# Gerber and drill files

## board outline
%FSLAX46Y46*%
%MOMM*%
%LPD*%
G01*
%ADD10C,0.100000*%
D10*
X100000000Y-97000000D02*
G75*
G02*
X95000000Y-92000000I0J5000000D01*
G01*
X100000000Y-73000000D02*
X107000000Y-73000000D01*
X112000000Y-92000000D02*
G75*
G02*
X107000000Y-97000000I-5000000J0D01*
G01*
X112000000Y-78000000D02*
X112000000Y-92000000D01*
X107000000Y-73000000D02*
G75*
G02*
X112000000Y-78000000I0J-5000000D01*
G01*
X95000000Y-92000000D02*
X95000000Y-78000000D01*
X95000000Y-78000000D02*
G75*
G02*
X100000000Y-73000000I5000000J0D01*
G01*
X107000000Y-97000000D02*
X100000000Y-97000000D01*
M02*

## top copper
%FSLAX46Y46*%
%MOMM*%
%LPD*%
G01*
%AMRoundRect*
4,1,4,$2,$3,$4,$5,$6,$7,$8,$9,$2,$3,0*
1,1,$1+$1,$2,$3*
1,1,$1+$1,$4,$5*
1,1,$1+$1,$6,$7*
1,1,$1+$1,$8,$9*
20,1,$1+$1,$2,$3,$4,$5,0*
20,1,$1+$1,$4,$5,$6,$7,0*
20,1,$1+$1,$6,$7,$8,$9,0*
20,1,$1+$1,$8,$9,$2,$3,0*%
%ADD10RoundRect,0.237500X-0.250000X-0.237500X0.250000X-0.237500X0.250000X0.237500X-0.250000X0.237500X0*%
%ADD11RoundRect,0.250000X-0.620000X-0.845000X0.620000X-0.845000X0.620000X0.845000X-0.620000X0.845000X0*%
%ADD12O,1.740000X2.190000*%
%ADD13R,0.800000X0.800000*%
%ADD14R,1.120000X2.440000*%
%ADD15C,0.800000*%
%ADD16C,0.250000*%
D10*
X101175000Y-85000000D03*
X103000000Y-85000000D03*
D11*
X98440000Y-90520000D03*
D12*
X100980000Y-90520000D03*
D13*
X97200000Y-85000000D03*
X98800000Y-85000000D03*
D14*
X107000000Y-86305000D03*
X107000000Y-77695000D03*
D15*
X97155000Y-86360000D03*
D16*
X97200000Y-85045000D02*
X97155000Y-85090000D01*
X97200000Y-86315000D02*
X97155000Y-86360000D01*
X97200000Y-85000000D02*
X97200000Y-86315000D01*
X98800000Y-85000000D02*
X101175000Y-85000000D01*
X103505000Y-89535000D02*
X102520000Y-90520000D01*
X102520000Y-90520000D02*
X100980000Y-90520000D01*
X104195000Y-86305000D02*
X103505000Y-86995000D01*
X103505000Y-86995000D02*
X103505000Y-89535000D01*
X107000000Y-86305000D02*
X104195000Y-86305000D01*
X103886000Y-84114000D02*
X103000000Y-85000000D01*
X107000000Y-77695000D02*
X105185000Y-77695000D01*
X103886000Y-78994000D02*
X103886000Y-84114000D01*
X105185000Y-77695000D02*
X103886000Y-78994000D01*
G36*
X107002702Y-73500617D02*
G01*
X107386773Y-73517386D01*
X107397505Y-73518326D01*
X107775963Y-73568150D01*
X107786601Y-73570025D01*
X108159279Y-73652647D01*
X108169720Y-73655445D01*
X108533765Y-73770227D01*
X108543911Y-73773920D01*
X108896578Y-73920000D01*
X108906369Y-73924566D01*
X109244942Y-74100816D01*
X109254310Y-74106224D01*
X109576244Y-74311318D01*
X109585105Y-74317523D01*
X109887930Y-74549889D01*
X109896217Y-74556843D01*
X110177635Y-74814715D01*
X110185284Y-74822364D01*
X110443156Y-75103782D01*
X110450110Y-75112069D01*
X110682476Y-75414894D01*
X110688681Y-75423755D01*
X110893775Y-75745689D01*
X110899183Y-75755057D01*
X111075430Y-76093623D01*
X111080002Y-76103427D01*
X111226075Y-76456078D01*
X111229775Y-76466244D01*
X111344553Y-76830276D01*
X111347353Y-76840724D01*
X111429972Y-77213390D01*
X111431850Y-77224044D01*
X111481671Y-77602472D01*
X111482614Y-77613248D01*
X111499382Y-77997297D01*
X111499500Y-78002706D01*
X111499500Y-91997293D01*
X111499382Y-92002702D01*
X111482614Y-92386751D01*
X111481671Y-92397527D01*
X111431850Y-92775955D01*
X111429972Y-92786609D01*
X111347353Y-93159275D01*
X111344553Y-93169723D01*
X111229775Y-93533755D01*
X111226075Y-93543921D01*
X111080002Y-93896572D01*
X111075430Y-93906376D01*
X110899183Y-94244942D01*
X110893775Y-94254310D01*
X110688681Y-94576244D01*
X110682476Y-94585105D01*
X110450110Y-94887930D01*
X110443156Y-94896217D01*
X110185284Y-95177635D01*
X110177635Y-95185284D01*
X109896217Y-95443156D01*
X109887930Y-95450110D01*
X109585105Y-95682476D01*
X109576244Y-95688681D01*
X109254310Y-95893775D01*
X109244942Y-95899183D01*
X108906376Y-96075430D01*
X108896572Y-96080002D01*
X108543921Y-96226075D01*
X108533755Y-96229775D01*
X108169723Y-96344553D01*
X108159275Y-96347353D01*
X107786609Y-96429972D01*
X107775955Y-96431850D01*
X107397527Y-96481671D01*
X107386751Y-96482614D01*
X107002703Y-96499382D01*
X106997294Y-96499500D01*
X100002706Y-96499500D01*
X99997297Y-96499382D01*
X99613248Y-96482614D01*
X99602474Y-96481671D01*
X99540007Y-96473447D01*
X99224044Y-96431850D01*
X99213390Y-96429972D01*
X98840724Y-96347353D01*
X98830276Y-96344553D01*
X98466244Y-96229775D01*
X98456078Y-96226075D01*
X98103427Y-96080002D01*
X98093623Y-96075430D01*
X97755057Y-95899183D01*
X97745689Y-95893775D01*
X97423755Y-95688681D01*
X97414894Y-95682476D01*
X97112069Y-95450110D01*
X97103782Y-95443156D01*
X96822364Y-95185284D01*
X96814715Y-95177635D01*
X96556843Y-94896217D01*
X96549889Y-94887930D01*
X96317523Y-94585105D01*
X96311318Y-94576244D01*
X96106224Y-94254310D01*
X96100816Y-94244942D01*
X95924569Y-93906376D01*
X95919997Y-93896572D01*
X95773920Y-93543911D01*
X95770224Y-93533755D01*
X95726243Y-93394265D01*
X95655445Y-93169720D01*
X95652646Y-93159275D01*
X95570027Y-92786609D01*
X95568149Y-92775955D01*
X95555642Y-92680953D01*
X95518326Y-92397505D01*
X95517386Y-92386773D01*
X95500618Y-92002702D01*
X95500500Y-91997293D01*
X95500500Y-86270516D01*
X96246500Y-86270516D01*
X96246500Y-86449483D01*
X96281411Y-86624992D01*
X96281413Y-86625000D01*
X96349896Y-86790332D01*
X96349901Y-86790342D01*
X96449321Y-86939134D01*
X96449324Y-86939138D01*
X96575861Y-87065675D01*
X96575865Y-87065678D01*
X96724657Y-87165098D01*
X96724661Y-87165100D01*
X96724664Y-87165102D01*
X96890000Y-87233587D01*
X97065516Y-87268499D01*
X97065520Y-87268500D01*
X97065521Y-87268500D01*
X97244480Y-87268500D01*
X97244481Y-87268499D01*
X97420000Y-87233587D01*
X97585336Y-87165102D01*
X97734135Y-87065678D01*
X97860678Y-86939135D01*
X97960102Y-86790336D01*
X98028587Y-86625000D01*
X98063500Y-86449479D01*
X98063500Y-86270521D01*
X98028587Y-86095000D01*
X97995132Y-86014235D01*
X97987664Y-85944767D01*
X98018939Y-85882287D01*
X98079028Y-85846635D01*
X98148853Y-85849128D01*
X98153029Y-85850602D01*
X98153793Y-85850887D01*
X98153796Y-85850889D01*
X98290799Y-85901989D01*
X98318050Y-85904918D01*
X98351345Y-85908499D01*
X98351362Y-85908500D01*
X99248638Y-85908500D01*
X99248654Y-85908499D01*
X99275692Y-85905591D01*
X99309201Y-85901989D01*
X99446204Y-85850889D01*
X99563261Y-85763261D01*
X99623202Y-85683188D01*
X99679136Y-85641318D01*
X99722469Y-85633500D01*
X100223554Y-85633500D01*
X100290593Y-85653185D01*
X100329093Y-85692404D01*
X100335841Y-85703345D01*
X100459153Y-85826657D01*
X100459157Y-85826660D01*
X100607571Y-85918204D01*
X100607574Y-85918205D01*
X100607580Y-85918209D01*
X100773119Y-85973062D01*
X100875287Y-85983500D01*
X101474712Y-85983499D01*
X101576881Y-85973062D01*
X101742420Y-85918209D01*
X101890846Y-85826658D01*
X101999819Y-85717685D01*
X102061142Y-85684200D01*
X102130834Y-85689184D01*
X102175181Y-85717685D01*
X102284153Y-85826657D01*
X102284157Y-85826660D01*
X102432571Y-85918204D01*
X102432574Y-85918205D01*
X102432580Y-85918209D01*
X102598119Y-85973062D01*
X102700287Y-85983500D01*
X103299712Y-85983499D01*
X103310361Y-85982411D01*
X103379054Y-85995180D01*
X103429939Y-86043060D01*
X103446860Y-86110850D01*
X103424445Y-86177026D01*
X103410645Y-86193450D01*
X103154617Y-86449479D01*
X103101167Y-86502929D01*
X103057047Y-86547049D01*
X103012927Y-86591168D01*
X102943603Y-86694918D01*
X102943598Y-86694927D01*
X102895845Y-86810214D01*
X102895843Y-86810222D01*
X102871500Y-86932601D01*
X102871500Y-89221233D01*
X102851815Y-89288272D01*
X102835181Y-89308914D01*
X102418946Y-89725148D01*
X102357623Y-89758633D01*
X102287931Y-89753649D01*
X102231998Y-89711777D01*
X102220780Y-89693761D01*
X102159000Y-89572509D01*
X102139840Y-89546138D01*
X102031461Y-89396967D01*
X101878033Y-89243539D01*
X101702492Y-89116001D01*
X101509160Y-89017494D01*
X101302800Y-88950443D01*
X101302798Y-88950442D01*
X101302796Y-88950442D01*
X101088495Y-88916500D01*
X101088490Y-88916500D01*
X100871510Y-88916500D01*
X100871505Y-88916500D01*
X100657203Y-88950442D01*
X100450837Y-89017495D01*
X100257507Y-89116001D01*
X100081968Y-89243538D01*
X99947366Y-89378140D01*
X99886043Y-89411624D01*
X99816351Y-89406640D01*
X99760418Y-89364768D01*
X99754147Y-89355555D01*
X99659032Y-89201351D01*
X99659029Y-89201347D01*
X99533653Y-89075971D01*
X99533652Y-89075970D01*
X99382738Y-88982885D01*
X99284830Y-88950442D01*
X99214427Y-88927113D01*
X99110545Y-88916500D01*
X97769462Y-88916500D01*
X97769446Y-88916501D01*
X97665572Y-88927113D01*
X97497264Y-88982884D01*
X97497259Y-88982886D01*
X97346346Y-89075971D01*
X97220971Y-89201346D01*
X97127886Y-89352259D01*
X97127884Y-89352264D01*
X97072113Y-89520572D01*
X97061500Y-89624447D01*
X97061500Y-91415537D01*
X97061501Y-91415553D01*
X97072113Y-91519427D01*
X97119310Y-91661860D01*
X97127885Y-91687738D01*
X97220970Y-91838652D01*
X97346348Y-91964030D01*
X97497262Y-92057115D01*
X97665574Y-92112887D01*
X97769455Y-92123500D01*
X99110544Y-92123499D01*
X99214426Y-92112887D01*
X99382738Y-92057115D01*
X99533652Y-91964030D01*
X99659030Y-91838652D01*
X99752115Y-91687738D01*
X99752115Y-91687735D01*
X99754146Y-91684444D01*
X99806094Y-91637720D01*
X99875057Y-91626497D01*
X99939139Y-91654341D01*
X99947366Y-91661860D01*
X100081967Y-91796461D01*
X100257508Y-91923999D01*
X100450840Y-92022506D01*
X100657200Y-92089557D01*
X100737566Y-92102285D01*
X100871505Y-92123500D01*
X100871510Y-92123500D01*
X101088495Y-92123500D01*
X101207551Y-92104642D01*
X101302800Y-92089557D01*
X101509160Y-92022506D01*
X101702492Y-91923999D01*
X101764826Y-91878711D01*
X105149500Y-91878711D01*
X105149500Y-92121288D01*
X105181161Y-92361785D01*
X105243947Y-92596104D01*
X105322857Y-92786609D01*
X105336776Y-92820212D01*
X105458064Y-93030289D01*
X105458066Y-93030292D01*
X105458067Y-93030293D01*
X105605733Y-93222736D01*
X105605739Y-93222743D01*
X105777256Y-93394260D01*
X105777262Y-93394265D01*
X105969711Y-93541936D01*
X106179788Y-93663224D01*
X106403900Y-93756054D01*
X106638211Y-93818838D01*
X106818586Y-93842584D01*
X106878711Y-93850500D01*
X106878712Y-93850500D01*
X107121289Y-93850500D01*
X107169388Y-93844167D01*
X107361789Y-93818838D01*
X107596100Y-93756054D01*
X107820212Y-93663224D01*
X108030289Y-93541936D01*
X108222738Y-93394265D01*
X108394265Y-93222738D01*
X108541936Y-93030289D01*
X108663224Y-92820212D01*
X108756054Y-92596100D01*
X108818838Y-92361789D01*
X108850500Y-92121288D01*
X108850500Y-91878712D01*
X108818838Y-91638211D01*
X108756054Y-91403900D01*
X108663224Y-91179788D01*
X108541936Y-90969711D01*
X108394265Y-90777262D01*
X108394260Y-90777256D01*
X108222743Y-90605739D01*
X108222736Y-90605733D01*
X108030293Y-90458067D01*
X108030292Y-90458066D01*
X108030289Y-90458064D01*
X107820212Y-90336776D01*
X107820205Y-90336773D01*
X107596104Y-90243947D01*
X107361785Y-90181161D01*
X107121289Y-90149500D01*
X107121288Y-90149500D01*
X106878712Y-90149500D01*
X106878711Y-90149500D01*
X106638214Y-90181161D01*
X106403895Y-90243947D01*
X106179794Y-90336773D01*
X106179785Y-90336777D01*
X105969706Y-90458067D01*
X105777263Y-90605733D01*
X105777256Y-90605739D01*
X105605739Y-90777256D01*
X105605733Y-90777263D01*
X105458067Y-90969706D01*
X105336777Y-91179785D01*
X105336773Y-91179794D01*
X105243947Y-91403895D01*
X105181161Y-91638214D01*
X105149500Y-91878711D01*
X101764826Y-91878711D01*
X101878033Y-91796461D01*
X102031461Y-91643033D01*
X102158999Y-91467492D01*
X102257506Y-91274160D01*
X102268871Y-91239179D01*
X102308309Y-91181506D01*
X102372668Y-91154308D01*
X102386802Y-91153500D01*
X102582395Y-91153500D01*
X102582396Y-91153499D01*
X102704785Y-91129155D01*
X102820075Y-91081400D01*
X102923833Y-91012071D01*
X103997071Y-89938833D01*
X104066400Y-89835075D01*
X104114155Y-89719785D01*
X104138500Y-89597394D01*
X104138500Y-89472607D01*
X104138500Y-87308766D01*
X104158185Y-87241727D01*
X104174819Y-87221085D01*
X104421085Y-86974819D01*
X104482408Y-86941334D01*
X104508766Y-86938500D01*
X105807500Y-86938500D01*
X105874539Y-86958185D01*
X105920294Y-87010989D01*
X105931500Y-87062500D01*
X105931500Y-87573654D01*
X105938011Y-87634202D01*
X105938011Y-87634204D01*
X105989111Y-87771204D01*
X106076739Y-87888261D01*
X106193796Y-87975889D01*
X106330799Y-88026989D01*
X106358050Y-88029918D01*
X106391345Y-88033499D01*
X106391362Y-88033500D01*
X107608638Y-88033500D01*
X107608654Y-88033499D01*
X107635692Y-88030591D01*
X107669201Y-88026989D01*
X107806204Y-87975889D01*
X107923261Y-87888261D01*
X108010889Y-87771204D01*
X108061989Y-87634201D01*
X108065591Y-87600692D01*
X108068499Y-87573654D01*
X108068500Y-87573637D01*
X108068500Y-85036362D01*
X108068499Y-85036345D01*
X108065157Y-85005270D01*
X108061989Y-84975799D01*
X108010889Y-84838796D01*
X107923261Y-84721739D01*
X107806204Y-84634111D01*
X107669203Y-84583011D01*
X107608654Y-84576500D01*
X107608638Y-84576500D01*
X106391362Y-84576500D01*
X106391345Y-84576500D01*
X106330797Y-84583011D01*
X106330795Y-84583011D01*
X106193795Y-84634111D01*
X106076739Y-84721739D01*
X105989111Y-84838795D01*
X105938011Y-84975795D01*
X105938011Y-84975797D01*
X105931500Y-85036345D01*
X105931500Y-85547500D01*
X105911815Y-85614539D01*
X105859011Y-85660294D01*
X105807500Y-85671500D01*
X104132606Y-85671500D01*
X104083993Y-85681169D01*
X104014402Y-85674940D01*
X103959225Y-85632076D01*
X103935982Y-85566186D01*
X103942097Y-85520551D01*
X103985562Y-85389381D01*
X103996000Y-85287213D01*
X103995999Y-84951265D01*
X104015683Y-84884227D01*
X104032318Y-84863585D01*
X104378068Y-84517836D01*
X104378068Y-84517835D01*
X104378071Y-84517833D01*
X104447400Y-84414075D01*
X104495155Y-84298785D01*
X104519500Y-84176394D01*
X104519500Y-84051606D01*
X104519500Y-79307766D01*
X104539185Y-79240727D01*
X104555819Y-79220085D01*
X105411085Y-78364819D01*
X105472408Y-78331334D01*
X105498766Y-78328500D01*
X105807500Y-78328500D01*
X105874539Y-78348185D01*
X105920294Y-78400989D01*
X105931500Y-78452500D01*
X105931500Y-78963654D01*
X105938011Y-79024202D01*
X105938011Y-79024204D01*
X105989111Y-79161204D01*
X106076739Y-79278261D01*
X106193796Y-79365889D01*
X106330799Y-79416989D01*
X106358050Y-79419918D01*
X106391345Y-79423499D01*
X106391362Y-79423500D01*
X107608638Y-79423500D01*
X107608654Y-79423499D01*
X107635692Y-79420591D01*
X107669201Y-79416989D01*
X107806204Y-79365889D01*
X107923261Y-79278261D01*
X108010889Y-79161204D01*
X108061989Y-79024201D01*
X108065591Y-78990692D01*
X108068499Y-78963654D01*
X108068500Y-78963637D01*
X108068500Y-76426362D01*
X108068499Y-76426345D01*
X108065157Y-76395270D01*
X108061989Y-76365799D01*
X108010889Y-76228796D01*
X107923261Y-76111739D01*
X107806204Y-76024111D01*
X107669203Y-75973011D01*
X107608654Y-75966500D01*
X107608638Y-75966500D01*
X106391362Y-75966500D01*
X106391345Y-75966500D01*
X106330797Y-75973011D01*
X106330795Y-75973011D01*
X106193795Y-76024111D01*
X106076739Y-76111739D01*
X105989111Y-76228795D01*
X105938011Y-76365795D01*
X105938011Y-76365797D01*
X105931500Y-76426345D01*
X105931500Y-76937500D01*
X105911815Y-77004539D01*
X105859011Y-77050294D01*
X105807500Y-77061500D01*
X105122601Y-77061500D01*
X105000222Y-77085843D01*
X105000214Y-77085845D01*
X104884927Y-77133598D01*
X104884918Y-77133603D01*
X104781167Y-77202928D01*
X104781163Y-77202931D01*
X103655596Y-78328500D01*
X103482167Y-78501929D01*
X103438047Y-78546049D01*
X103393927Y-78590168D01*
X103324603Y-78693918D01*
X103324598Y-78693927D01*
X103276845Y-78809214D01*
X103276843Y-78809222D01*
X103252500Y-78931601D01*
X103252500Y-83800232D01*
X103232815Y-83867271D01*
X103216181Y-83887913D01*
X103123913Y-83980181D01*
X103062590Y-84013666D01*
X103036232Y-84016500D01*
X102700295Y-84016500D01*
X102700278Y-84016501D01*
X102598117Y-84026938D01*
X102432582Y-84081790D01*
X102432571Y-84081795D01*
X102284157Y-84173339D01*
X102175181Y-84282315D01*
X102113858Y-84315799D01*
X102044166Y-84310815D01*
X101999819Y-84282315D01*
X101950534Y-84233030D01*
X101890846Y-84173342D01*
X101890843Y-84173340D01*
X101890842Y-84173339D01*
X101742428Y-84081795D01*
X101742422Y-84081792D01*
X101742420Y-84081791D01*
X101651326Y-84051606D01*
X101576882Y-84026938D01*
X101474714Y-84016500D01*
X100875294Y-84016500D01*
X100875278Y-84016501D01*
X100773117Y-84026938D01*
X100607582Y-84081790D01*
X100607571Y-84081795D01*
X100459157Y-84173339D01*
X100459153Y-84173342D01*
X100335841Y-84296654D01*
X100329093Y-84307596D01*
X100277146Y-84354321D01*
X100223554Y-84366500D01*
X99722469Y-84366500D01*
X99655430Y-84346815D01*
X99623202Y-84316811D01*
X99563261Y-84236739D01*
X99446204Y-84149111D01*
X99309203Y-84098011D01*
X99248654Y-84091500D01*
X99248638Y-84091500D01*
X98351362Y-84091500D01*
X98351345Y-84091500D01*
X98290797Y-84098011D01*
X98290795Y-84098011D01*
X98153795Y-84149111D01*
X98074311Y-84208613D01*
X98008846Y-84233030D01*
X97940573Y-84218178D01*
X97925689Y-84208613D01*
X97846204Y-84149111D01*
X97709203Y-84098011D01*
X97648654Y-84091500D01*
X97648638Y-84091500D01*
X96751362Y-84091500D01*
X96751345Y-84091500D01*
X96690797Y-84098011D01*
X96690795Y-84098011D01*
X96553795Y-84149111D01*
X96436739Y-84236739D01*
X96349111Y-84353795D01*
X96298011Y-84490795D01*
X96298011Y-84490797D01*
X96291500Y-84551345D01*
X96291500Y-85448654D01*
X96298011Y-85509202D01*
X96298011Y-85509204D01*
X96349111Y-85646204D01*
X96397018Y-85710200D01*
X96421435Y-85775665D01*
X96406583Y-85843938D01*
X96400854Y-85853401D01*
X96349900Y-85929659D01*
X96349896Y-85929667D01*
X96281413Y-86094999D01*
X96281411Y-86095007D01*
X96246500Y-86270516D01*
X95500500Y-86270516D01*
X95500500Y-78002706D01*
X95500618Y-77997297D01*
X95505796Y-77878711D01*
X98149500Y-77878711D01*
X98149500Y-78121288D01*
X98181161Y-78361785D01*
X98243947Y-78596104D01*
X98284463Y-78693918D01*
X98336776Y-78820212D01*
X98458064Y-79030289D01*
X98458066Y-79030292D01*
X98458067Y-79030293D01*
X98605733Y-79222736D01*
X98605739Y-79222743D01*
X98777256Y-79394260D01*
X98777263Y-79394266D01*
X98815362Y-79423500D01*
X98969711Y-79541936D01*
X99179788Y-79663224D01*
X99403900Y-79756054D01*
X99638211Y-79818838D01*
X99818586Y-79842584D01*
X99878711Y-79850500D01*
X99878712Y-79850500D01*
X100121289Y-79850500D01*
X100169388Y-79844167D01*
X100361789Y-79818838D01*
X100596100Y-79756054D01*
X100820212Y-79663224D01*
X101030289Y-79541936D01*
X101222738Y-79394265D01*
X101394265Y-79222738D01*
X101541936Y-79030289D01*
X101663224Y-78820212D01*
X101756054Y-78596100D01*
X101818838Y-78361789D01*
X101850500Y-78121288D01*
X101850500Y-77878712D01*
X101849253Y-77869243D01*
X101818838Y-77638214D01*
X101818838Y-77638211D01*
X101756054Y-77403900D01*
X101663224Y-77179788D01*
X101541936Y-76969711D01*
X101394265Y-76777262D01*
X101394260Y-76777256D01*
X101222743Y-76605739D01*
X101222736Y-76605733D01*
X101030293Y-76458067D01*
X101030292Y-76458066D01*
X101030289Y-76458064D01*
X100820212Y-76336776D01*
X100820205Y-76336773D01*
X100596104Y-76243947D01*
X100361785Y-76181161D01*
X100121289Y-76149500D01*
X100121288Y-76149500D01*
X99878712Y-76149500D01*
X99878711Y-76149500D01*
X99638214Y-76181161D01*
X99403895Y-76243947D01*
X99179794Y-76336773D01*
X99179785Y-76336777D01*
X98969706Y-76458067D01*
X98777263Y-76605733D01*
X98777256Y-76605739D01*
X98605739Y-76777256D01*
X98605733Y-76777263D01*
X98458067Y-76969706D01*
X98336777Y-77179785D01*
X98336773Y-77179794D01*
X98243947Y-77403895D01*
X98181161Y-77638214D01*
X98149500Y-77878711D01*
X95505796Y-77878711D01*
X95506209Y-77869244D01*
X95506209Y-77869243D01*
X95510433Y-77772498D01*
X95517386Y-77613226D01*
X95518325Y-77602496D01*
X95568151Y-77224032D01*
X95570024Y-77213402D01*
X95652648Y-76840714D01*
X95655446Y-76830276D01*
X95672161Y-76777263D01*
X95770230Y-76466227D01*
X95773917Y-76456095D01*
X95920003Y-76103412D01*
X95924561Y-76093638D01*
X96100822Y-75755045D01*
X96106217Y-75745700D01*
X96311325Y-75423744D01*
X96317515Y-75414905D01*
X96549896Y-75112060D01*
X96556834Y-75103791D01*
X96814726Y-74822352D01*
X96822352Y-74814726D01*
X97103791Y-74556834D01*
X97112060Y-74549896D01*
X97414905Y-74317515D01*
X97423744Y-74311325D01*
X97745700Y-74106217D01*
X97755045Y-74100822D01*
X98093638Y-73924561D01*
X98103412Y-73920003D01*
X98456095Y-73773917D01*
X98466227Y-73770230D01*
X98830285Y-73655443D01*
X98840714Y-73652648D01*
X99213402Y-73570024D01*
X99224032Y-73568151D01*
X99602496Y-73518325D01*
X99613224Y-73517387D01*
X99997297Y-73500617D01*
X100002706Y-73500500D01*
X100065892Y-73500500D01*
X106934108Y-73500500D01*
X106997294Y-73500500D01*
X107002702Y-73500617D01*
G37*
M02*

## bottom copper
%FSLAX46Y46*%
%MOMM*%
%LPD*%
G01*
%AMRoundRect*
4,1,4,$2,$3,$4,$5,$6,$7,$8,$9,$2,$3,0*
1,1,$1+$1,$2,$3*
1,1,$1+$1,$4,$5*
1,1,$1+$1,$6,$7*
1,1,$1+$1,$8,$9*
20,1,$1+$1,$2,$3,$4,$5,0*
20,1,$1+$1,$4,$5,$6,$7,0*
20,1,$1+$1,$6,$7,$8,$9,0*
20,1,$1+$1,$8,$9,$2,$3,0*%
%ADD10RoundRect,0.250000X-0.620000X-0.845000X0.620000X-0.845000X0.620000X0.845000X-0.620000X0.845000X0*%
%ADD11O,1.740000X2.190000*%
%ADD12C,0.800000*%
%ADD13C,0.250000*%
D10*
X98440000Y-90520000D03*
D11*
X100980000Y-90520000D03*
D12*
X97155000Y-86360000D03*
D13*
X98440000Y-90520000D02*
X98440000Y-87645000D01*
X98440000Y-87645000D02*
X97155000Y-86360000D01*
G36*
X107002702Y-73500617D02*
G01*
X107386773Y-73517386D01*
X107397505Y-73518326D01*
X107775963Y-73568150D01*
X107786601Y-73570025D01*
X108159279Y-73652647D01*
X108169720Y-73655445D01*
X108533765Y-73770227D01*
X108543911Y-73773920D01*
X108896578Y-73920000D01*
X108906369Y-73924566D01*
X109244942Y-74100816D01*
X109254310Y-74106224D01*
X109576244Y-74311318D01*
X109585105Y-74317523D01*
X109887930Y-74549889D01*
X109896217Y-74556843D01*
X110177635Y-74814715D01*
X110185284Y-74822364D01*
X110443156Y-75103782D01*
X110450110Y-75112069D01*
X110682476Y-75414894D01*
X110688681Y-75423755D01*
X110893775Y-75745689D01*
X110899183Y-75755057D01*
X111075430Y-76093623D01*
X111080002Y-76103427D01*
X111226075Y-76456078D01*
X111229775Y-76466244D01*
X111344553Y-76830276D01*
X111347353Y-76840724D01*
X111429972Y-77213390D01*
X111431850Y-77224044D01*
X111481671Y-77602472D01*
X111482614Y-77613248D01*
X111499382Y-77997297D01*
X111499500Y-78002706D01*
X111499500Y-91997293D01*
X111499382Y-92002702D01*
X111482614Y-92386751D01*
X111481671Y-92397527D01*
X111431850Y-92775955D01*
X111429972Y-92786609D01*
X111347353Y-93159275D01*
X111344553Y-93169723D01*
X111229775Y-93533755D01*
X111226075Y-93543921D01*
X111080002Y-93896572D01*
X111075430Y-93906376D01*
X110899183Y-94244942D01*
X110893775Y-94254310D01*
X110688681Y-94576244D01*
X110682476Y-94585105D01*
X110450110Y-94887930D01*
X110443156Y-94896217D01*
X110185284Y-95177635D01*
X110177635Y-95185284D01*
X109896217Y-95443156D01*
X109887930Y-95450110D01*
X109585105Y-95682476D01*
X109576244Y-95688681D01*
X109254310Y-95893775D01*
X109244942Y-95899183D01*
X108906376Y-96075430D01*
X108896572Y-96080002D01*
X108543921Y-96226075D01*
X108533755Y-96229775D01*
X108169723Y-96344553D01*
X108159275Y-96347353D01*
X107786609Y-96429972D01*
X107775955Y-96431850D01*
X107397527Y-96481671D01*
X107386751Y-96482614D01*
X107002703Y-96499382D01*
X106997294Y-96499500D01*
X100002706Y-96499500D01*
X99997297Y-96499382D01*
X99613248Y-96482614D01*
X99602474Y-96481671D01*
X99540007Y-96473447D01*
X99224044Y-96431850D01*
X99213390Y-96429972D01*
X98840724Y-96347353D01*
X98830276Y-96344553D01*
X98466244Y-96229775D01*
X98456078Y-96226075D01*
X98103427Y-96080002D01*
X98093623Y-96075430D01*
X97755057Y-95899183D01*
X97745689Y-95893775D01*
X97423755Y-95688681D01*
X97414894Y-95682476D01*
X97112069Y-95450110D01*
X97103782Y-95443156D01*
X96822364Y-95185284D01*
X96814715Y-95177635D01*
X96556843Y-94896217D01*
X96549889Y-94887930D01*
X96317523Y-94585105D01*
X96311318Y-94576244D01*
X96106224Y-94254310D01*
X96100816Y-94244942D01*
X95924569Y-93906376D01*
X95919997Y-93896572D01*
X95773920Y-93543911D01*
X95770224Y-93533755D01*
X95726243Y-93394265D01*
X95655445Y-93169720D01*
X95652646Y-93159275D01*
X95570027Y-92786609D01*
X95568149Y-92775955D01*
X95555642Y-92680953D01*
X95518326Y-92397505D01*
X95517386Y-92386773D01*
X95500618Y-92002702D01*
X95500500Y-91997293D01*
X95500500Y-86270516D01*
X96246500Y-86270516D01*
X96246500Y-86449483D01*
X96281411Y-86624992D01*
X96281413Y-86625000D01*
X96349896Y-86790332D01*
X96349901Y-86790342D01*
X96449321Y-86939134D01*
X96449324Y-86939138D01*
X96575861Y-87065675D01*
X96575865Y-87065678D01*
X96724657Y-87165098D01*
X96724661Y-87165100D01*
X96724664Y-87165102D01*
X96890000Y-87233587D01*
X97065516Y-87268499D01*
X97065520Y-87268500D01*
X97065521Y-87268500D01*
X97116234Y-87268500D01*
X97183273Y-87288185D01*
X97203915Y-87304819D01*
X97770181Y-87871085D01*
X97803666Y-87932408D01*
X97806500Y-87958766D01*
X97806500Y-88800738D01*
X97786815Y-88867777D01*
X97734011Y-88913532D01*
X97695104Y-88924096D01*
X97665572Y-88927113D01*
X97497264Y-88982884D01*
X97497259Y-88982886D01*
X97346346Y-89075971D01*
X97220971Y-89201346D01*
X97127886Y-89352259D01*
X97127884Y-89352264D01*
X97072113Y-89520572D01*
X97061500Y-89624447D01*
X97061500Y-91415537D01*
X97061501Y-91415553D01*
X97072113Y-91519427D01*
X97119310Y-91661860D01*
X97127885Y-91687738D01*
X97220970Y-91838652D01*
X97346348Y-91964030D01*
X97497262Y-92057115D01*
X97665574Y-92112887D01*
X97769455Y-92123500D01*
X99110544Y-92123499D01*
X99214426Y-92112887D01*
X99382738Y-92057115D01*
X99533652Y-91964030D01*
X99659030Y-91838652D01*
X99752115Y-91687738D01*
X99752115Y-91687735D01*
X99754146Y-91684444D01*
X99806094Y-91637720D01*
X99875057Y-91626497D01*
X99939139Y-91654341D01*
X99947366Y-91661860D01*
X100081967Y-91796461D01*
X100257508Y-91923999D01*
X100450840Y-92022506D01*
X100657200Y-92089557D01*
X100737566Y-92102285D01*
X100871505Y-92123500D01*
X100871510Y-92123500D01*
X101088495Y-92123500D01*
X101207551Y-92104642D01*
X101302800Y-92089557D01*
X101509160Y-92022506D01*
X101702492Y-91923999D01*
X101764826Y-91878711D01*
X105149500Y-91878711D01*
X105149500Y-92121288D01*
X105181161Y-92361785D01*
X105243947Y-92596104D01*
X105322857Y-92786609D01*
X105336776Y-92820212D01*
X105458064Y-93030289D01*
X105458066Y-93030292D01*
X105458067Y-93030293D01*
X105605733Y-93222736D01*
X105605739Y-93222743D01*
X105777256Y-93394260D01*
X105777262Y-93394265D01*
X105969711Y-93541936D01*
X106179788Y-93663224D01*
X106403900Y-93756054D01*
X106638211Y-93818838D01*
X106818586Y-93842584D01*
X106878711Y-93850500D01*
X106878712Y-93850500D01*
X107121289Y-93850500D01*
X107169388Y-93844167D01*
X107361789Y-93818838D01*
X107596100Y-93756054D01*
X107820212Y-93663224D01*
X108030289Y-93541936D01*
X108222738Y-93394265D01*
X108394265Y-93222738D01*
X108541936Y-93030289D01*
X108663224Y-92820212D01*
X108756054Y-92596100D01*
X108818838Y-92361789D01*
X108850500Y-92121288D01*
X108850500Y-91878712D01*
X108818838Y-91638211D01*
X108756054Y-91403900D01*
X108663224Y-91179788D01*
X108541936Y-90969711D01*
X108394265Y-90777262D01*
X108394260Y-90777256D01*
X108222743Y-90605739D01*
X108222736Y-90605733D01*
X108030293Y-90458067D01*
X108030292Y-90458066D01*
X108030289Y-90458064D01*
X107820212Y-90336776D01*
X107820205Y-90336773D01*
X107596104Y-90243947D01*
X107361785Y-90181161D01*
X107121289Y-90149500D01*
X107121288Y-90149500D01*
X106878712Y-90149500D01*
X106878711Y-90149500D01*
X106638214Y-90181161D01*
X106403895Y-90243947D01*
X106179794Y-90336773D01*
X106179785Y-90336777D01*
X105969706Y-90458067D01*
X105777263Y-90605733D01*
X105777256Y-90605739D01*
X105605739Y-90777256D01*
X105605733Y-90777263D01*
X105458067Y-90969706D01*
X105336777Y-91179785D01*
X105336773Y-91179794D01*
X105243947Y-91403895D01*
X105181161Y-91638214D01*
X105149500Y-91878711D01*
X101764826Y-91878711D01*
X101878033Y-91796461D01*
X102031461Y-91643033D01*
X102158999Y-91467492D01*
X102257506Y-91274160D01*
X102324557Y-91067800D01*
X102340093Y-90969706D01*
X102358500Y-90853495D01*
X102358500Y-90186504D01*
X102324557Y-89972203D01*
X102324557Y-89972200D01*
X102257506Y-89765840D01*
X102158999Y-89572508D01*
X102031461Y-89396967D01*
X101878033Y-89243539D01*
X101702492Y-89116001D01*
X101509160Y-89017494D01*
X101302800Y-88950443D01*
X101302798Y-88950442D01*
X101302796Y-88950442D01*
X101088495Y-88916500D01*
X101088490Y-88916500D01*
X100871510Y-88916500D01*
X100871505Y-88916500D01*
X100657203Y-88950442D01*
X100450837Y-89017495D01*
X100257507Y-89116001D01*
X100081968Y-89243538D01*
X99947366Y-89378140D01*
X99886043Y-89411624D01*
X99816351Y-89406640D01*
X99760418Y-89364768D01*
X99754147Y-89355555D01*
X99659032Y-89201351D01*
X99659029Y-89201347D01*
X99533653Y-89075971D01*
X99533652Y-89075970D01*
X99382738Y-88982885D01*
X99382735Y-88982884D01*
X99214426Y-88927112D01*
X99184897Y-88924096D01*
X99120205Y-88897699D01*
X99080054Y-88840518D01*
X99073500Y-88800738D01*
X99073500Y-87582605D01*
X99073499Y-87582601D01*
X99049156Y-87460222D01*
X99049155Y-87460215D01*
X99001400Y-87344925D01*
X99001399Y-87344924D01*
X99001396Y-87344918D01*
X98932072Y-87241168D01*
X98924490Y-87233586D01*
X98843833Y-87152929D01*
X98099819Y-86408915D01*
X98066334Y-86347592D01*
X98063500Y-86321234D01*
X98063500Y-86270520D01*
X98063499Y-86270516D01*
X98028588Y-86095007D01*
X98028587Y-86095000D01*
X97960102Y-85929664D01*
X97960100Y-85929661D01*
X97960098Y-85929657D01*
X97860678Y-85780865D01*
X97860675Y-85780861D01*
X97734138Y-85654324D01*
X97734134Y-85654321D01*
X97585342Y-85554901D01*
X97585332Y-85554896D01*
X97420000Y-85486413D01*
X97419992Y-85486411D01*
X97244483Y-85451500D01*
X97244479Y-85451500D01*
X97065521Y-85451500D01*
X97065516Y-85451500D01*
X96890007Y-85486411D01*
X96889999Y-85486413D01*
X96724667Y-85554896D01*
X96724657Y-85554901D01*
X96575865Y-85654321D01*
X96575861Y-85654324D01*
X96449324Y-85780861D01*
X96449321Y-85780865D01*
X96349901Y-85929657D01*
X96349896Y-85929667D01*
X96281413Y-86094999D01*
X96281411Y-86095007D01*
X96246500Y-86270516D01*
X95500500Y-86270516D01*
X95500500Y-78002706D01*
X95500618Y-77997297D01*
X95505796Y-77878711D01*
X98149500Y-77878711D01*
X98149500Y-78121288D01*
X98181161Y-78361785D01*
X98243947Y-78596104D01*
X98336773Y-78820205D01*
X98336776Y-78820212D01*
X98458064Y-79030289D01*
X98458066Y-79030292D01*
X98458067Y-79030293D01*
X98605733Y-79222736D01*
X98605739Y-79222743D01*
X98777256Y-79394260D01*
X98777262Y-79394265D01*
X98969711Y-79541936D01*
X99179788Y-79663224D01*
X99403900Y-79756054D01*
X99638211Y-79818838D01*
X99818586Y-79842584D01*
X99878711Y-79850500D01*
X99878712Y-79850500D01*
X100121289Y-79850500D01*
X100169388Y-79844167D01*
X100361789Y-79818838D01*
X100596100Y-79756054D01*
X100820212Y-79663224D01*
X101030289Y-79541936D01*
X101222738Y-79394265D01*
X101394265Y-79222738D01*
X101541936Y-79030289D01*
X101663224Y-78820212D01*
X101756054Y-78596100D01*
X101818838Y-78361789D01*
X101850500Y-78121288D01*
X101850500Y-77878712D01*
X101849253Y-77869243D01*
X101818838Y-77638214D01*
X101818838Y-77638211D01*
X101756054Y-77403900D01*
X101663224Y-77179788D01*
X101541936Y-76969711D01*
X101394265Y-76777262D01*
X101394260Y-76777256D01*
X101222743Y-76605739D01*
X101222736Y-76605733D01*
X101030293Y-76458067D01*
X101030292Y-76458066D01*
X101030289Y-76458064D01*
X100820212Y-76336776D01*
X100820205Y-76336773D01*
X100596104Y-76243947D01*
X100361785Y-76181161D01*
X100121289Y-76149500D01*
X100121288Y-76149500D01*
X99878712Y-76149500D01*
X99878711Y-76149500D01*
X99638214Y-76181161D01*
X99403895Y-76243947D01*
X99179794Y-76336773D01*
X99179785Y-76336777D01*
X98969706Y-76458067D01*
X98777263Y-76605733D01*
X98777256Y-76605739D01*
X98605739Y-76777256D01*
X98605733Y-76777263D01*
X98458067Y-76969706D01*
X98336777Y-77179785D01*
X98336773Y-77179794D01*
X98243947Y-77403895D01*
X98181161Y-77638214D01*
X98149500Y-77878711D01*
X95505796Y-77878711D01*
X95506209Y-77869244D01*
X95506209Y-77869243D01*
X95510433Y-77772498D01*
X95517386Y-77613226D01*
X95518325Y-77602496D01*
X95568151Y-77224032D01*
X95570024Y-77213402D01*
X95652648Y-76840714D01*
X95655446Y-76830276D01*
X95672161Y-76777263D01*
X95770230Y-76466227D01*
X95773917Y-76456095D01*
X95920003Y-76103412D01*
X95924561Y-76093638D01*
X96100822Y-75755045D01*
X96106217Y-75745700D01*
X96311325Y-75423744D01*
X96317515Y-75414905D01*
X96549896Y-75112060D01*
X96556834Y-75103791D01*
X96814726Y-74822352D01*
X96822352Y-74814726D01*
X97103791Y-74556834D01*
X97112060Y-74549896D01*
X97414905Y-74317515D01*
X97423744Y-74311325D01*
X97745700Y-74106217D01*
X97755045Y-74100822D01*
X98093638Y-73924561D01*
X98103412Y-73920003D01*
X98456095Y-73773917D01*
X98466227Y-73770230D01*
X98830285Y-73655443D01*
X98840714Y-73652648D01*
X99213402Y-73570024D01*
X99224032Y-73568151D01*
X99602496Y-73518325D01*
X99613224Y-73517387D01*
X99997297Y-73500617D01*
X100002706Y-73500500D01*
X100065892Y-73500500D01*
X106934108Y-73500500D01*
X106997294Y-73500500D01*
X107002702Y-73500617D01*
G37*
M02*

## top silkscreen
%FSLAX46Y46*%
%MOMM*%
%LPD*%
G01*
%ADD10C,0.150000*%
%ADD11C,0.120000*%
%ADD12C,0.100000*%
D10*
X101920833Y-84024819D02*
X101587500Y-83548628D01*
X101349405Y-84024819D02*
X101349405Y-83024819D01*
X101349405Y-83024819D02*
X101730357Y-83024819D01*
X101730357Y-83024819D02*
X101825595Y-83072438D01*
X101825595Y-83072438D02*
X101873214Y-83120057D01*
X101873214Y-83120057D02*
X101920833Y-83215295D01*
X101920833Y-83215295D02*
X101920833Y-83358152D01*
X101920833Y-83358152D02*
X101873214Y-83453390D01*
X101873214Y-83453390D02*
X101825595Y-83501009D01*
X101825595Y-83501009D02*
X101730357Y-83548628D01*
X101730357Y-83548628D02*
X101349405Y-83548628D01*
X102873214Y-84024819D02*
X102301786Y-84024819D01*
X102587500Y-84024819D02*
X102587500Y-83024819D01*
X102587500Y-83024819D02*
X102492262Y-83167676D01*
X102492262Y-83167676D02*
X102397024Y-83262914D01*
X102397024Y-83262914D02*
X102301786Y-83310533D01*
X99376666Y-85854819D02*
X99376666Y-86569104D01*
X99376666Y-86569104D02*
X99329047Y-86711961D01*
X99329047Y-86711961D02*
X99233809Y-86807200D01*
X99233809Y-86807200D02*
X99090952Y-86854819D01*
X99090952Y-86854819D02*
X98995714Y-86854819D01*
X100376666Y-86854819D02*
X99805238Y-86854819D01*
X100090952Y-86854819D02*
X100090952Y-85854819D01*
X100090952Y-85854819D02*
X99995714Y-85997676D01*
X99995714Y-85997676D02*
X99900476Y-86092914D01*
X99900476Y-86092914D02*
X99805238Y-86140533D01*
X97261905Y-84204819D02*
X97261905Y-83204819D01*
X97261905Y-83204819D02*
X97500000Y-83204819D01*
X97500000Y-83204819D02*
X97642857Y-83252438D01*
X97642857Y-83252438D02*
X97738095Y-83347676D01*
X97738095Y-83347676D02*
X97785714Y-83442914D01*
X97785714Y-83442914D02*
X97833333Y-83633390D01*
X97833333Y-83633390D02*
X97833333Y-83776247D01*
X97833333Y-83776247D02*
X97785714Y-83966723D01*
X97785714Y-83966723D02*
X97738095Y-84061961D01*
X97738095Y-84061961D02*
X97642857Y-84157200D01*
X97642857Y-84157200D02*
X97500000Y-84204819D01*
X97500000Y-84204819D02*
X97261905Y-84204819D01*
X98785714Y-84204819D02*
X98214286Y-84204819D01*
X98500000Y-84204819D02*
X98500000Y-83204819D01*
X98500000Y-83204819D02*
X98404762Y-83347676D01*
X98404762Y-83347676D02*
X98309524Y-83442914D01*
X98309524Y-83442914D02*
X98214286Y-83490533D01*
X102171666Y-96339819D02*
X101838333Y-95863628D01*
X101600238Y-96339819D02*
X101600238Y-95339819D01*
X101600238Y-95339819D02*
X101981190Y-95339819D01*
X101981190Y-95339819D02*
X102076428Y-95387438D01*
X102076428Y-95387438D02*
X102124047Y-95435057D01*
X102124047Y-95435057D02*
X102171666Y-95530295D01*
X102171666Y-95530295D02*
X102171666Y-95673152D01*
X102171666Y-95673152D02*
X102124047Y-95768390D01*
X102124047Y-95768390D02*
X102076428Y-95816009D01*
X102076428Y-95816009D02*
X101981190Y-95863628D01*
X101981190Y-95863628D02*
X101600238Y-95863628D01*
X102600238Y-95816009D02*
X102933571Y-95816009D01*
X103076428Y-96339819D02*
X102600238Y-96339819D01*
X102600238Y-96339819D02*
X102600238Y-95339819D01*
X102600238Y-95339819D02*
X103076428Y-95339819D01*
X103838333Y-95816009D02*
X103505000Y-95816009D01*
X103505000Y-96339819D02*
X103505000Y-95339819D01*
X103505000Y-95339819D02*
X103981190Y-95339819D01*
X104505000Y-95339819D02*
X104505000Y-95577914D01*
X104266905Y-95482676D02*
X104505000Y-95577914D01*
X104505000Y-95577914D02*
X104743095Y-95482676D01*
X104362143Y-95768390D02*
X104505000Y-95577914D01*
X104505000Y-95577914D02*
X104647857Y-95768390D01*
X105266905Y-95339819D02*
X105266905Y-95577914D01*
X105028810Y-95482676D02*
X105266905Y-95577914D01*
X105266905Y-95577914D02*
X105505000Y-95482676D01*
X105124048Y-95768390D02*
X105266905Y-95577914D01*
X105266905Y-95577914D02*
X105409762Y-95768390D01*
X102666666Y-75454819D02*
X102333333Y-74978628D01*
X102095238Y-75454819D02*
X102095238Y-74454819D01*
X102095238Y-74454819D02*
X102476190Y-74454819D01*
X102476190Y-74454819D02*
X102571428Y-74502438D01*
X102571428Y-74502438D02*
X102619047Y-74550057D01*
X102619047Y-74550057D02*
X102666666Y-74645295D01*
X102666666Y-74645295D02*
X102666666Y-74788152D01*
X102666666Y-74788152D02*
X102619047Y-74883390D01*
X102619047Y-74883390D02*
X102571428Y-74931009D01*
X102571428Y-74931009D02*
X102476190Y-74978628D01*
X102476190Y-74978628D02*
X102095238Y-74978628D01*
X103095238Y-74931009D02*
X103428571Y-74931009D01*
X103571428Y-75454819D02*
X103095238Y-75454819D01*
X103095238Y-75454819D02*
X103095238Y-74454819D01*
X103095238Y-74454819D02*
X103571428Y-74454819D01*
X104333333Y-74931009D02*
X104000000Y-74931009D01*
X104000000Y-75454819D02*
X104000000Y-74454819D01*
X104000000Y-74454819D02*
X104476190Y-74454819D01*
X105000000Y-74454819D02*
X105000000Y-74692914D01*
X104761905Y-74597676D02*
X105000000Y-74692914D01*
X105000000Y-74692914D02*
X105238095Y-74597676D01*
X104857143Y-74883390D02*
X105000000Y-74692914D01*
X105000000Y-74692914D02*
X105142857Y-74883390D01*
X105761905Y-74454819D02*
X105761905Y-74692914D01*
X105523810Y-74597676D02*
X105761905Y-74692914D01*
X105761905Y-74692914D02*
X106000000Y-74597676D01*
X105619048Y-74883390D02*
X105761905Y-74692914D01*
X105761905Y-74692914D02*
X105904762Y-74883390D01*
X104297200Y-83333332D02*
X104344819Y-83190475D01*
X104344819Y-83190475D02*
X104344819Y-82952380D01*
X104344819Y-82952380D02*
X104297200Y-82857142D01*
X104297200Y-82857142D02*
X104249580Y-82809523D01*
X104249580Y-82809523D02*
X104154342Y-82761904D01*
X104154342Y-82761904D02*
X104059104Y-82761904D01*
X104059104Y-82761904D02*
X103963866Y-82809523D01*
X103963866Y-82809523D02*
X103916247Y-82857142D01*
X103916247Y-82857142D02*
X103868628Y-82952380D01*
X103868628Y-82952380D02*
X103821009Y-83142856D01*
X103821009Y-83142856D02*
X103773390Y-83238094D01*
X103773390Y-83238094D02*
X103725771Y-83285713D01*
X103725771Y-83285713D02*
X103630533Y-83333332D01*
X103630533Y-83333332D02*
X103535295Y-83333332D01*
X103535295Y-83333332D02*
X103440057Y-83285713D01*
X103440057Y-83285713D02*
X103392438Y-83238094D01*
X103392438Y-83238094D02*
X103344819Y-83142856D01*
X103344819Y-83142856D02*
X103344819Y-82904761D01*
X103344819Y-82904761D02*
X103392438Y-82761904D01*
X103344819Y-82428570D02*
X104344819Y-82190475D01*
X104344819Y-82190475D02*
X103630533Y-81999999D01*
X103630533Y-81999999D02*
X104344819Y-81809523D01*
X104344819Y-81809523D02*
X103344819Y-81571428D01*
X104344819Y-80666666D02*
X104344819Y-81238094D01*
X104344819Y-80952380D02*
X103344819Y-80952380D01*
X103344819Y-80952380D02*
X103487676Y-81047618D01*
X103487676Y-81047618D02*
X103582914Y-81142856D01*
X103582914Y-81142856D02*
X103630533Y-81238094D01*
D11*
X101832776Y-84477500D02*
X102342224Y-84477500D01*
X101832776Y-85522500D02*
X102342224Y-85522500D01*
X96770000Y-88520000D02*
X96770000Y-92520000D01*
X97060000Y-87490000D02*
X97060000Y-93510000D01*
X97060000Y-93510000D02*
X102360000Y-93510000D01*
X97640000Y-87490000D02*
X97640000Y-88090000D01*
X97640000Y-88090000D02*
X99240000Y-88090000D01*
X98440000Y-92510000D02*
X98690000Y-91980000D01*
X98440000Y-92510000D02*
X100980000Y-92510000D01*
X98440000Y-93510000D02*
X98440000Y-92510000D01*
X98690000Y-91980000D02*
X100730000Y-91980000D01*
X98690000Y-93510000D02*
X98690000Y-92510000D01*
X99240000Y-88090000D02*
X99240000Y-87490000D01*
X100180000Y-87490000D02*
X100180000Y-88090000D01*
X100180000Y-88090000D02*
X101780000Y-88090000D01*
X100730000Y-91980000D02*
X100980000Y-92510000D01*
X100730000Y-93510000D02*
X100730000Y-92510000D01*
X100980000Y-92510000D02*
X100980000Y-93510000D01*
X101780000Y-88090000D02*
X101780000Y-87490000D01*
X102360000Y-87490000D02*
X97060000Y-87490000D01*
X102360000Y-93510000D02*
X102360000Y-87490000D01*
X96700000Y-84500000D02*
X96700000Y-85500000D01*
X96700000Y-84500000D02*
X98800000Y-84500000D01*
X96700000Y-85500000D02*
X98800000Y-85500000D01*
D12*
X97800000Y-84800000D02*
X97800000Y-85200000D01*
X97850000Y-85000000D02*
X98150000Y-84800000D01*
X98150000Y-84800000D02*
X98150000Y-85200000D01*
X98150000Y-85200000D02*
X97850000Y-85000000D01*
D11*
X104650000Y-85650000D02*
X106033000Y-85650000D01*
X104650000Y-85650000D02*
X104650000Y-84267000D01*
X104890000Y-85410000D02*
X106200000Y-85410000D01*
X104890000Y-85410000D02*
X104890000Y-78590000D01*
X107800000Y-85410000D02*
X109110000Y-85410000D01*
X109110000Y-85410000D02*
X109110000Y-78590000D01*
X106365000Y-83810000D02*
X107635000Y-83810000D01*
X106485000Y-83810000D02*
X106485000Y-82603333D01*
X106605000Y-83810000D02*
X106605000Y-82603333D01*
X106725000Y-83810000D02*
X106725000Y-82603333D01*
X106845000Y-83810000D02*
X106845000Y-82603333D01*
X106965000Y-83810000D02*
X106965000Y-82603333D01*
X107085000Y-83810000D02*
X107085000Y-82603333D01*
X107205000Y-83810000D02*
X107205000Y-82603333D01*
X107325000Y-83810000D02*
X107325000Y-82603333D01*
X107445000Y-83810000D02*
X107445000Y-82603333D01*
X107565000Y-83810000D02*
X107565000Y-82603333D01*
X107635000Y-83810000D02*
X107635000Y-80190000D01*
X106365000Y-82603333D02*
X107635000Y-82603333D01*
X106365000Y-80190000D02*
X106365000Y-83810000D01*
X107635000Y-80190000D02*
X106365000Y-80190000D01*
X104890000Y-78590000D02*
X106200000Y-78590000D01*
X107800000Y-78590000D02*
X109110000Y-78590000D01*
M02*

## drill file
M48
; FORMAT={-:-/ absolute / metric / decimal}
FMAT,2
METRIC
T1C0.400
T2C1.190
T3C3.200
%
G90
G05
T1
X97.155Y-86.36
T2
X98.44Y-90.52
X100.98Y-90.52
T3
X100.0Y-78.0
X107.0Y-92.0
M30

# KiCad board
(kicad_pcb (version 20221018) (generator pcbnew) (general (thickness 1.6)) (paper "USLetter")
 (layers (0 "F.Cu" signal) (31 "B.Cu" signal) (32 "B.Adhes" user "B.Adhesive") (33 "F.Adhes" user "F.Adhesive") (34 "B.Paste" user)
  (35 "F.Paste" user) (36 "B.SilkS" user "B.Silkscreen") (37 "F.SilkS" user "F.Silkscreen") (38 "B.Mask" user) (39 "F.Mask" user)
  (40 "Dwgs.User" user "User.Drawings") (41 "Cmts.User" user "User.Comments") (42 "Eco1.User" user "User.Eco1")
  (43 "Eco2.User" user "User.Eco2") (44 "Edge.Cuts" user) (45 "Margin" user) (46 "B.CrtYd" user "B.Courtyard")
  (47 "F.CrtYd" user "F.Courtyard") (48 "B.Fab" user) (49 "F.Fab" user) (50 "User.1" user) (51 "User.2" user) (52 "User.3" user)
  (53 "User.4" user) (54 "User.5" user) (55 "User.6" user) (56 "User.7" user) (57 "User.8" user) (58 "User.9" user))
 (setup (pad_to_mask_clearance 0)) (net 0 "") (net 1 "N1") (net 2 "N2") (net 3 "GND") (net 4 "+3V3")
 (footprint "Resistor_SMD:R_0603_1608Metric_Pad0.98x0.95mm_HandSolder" (layer "F.Cu") (at 102.0875 85)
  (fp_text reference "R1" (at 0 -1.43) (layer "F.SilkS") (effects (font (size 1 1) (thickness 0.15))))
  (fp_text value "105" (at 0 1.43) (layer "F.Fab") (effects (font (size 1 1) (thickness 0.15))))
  (fp_line (start -0.254724 -0.5225) (end 0.254724 -0.5225) (stroke (width 0.12) (type solid)) (layer "F.SilkS"))
  (fp_line (start -0.254724 0.5225) (end 0.254724 0.5225) (stroke (width 0.12) (type solid)) (layer "F.SilkS"))
  (pad "1" smd roundrect (at -0.9125 0) (size 0.975 0.95) (layers "F.Cu" "F.Paste" "F.Mask") (roundrect_rratio 0.25) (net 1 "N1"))
  (pad "2" smd roundrect (at 0.9125 0) (size 0.975 0.95) (layers "F.Cu" "F.Paste" "F.Mask") (roundrect_rratio 0.25) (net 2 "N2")))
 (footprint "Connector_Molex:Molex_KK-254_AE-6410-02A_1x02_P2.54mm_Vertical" (layer "F.Cu") (at 98.44 90.52)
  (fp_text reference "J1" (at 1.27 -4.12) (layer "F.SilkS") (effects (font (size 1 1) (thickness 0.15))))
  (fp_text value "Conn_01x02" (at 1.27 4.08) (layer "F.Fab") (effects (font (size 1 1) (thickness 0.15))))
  (fp_line (start -1.67 -2) (end -1.67 2) (stroke (width 0.12) (type solid)) (layer "F.SilkS"))
  (fp_line (start -1.38 -3.03) (end -1.38 2.99) (stroke (width 0.12) (type solid)) (layer "F.SilkS"))
  (fp_line (start -1.38 2.99) (end 3.92 2.99) (stroke (width 0.12) (type solid)) (layer "F.SilkS"))
  (fp_line (start -0.8 -3.03) (end -0.8 -2.43) (stroke (width 0.12) (type solid)) (layer "F.SilkS"))
  (fp_line (start -0.8 -2.43) (end 0.8 -2.43) (stroke (width 0.12) (type solid)) (layer "F.SilkS"))
  (fp_line (start 0 1.99) (end 0.25 1.46) (stroke (width 0.12) (type solid)) (layer "F.SilkS"))
  (fp_line (start 0 1.99) (end 2.54 1.99) (stroke (width 0.12) (type solid)) (layer "F.SilkS"))
  (fp_line (start 0 2.99) (end 0 1.99) (stroke (width 0.12) (type solid)) (layer "F.SilkS"))
  (fp_line (start 0.25 1.46) (end 2.29 1.46) (stroke (width 0.12) (type solid)) (layer "F.SilkS"))
  (fp_line (start 0.25 2.99) (end 0.25 1.99) (stroke (width 0.12) (type solid)) (layer "F.SilkS"))
  (fp_line (start 0.8 -2.43) (end 0.8 -3.03) (stroke (width 0.12) (type solid)) (layer "F.SilkS"))
  (fp_line (start 1.74 -3.03) (end 1.74 -2.43) (stroke (width 0.12) (type solid)) (layer "F.SilkS"))
  (fp_line (start 1.74 -2.43) (end 3.34 -2.43) (stroke (width 0.12) (type solid)) (layer "F.SilkS"))
  (fp_line (start 2.29 1.46) (end 2.54 1.99) (stroke (width 0.12) (type solid)) (layer "F.SilkS"))
  (fp_line (start 2.29 2.99) (end 2.29 1.99) (stroke (width 0.12) (type solid)) (layer "F.SilkS"))
  (fp_line (start 2.54 1.99) (end 2.54 2.99) (stroke (width 0.12) (type solid)) (layer "F.SilkS"))
  (fp_line (start 3.34 -2.43) (end 3.34 -3.03) (stroke (width 0.12) (type solid)) (layer "F.SilkS"))
  (fp_line (start 3.92 -3.03) (end -1.38 -3.03) (stroke (width 0.12) (type solid)) (layer "F.SilkS"))
  (fp_line (start 3.92 2.99) (end 3.92 -3.03) (stroke (width 0.12) (type solid)) (layer "F.SilkS"))
  (pad "1" thru_hole roundrect (at 0 0) (size 1.74 2.19) (drill 1.19) (layers "*.Cu" "*.Mask") (roundrect_rratio 0.143678) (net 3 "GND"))
  (pad "2" thru_hole oval (at 2.54 0) (size 1.74 2.19) (drill 1.19) (layers "*.Cu" "*.Mask") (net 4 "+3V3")))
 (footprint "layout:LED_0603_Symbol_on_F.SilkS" (layer "F.Cu") (at 98 85)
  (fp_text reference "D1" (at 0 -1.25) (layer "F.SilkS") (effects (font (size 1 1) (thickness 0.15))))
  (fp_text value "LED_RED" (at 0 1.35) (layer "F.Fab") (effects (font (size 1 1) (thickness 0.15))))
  (fp_line (start -1.3 -0.5) (end -1.3 0.5) (stroke (width 0.12) (type solid)) (layer "F.SilkS"))
  (fp_line (start -1.3 -0.5) (end 0.8 -0.5) (stroke (width 0.12) (type solid)) (layer "F.SilkS"))
  (fp_line (start -1.3 0.5) (end 0.8 0.5) (stroke (width 0.12) (type solid)) (layer "F.SilkS"))
  (fp_line (start -0.2 -0.2) (end -0.2 0.2) (stroke (width 0.1) (type solid)) (layer "F.SilkS"))
  (fp_line (start -0.15 0) (end 0.15 -0.2) (stroke (width 0.1) (type solid)) (layer "F.SilkS"))
  (fp_line (start 0.15 -0.2) (end 0.15 0.2) (stroke (width 0.1) (type solid)) (layer "F.SilkS"))
  (fp_line (start 0.15 0.2) (end -0.15 0) (stroke (width 0.1) (type solid)) (layer "F.SilkS"))
  (pad "1" smd rect (at -0.8 0 180) (size 0.8 0.8) (layers "F.Cu" "F.Paste" "F.Mask") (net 3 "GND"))
  (pad "2" smd rect (at 0.8 0 180) (size 0.8 0.8) (layers "F.Cu" "F.Paste" "F.Mask") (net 1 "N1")))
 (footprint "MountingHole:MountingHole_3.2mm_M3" (layer "F.Cu") (at 107 92)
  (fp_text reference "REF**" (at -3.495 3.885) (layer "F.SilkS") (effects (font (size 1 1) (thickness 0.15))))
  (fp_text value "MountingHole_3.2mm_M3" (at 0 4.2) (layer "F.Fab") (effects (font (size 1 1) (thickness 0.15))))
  (pad "" np_thru_hole circle (at 0 0) (size 3.2 3.2) (drill 3.2) (layers "F&B.Cu" "*.Mask")))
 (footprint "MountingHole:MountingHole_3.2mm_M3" (layer "F.Cu") (at 100 78)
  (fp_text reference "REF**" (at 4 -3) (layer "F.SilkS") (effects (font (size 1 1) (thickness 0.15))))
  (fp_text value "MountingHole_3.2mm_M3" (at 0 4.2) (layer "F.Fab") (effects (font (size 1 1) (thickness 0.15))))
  (pad "" np_thru_hole circle (at 0 0) (size 3.2 3.2) (drill 3.2) (layers "*.Cu" "*.Mask")))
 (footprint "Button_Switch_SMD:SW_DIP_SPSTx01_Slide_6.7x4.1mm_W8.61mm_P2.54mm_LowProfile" (layer "F.Cu") (at 107 82 90)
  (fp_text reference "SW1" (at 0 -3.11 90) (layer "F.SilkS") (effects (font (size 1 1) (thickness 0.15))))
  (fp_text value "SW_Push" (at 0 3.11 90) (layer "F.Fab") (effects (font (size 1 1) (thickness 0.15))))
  (fp_line (start -3.65 -2.35) (end -3.65 -0.967) (stroke (width 0.12) (type solid)) (layer "F.SilkS"))
  (fp_line (start -3.65 -2.35) (end -2.267 -2.35) (stroke (width 0.12) (type solid)) (layer "F.SilkS"))
  (fp_line (start -3.41 -2.11) (end -3.41 -0.8) (stroke (width 0.12) (type solid)) (layer "F.SilkS"))
  (fp_line (start -3.41 -2.11) (end 3.41 -2.11) (stroke (width 0.12) (type solid)) (layer "F.SilkS"))
  (fp_line (start -3.41 0.8) (end -3.41 2.11) (stroke (width 0.12) (type solid)) (layer "F.SilkS"))
  (fp_line (start -3.41 2.11) (end 3.41 2.11) (stroke (width 0.12) (type solid)) (layer "F.SilkS"))
  (fp_line (start -1.81 -0.635) (end -1.81 0.635) (stroke (width 0.12) (type solid)) (layer "F.SilkS"))
  (fp_line (start -1.81 -0.515) (end -0.603333 -0.515) (stroke (width 0.12) (type solid)) (layer "F.SilkS"))
  (fp_line (start -1.81 -0.395) (end -0.603333 -0.395) (stroke (width 0.12) (type solid)) (layer "F.SilkS"))
  (fp_line (start -1.81 -0.275) (end -0.603333 -0.275) (stroke (width 0.12) (type solid)) (layer "F.SilkS"))
  (fp_line (start -1.81 -0.155) (end -0.603333 -0.155) (stroke (width 0.12) (type solid)) (layer "F.SilkS"))
  (fp_line (start -1.81 -0.035) (end -0.603333 -0.035) (stroke (width 0.12) (type solid)) (layer "F.SilkS"))
  (fp_line (start -1.81 0.085) (end -0.603333 0.085) (stroke (width 0.12) (type solid)) (layer "F.SilkS"))
  (fp_line (start -1.81 0.205) (end -0.603333 0.205) (stroke (width 0.12) (type solid)) (layer "F.SilkS"))
  (fp_line (start -1.81 0.325) (end -0.603333 0.325) (stroke (width 0.12) (type solid)) (layer "F.SilkS"))
  (fp_line (start -1.81 0.445) (end -0.603333 0.445) (stroke (width 0.12) (type solid)) (layer "F.SilkS"))
  (fp_line (start -1.81 0.565) (end -0.603333 0.565) (stroke (width 0.12) (type solid)) (layer "F.SilkS"))
  (fp_line (start -1.81 0.635) (end 1.81 0.635) (stroke (width 0.12) (type solid)) (layer "F.SilkS"))
  (fp_line (start -0.603333 -0.635) (end -0.603333 0.635) (stroke (width 0.12) (type solid)) (layer "F.SilkS"))
  (fp_line (start 1.81 -0.635) (end -1.81 -0.635) (stroke (width 0.12) (type solid)) (layer "F.SilkS"))
  (fp_line (start 1.81 0.635) (end 1.81 -0.635) (stroke (width 0.12) (type solid)) (layer "F.SilkS"))
  (fp_line (start 3.41 -2.11) (end 3.41 -0.8) (stroke (width 0.12) (type solid)) (layer "F.SilkS"))
  (fp_line (start 3.41 0.8) (end 3.41 2.11) (stroke (width 0.12) (type solid)) (layer "F.SilkS"))
  (pad "1" smd rect (at -4.305 0 90) (size 2.44 1.12) (layers "F.Cu" "F.Paste" "F.Mask") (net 4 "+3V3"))
  (pad "2" smd rect (at 4.305 0 90) (size 2.44 1.12) (layers "F.Cu" "F.Paste" "F.Mask") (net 2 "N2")))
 (gr_arc (start 100 97) (mid 96.464466 95.535534) (end 95 92) (stroke (width 0.1) (type default)) (layer "Edge.Cuts"))
 (gr_line (start 100 73) (end 107 73) (stroke (width 0.1) (type default)) (layer "Edge.Cuts"))
 (gr_arc (start 112 92) (mid 110.535534 95.535534) (end 107 97) (stroke (width 0.1) (type default)) (layer "Edge.Cuts"))
 (gr_line (start 112 78) (end 112 92) (stroke (width 0.1) (type default)) (layer "Edge.Cuts"))
 (gr_arc (start 107 73) (mid 110.535534 74.464466) (end 112 78) (stroke (width 0.1) (type default)) (layer "Edge.Cuts"))
 (gr_line (start 95 92) (end 95 78) (stroke (width 0.1) (type default)) (layer "Edge.Cuts"))
 (gr_arc (start 95 78) (mid 96.464466 74.464466) (end 100 73) (stroke (width 0.1) (type default)) (layer "Edge.Cuts"))
 (gr_line (start 107 97) (end 100 97) (stroke (width 0.1) (type default)) (layer "Edge.Cuts"))
 (segment (start 97.2 85.045) (end 97.155 85.09) (width 0.25) (layer "F.Cu") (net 3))
 (segment (start 97.2 86.315) (end 97.155 86.36) (width 0.25) (layer "F.Cu") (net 3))
 (segment (start 97.2 85) (end 97.2 86.315) (width 0.25) (layer "F.Cu") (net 3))
 (via (at 97.155 86.36) (size 0.8) (drill 0.4) (layers "F.Cu" "B.Cu") (free) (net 3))
 (segment (start 98.44 90.52) (end 98.44 87.645) (width 0.25) (layer "B.Cu") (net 3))
 (segment (start 98.44 87.645) (end 97.155 86.36) (width 0.25) (layer "B.Cu") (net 3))
 (segment (start 98.8 85) (end 101.175 85) (width 0.25) (layer "F.Cu") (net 1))
 (segment (start 103.505 89.535) (end 102.52 90.52) (width 0.25) (layer "F.Cu") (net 4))
 (segment (start 102.52 90.52) (end 100.98 90.52) (width 0.25) (layer "F.Cu") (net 4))
 (segment (start 104.195 86.305) (end 103.505 86.995) (width 0.25) (layer "F.Cu") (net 4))
 (segment (start 103.505 86.995) (end 103.505 89.535) (width 0.25) (layer "F.Cu") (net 4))
 (segment (start 107 86.305) (end 104.195 86.305) (width 0.25) (layer "F.Cu") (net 4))
 (segment (start 103.886 84.114) (end 103 85) (width 0.25) (layer "F.Cu") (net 2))
 (segment (start 107 77.695) (end 105.185 77.695) (width 0.25) (layer "F.Cu") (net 2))
 (segment (start 103.886 78.994) (end 103.886 84.114) (width 0.25) (layer "F.Cu") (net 2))
 (segment (start 105.185 77.695) (end 103.886 78.994) (width 0.25) (layer "F.Cu") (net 2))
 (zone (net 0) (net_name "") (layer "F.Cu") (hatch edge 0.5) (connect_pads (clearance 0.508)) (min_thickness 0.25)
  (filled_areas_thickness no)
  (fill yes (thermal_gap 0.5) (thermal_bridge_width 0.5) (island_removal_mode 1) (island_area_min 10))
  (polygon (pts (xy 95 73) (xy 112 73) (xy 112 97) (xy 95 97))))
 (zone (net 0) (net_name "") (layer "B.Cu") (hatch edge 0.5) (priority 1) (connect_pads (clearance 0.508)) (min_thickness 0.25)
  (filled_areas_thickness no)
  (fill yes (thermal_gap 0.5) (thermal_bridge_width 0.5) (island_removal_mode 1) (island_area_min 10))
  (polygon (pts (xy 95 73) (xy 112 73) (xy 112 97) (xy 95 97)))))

